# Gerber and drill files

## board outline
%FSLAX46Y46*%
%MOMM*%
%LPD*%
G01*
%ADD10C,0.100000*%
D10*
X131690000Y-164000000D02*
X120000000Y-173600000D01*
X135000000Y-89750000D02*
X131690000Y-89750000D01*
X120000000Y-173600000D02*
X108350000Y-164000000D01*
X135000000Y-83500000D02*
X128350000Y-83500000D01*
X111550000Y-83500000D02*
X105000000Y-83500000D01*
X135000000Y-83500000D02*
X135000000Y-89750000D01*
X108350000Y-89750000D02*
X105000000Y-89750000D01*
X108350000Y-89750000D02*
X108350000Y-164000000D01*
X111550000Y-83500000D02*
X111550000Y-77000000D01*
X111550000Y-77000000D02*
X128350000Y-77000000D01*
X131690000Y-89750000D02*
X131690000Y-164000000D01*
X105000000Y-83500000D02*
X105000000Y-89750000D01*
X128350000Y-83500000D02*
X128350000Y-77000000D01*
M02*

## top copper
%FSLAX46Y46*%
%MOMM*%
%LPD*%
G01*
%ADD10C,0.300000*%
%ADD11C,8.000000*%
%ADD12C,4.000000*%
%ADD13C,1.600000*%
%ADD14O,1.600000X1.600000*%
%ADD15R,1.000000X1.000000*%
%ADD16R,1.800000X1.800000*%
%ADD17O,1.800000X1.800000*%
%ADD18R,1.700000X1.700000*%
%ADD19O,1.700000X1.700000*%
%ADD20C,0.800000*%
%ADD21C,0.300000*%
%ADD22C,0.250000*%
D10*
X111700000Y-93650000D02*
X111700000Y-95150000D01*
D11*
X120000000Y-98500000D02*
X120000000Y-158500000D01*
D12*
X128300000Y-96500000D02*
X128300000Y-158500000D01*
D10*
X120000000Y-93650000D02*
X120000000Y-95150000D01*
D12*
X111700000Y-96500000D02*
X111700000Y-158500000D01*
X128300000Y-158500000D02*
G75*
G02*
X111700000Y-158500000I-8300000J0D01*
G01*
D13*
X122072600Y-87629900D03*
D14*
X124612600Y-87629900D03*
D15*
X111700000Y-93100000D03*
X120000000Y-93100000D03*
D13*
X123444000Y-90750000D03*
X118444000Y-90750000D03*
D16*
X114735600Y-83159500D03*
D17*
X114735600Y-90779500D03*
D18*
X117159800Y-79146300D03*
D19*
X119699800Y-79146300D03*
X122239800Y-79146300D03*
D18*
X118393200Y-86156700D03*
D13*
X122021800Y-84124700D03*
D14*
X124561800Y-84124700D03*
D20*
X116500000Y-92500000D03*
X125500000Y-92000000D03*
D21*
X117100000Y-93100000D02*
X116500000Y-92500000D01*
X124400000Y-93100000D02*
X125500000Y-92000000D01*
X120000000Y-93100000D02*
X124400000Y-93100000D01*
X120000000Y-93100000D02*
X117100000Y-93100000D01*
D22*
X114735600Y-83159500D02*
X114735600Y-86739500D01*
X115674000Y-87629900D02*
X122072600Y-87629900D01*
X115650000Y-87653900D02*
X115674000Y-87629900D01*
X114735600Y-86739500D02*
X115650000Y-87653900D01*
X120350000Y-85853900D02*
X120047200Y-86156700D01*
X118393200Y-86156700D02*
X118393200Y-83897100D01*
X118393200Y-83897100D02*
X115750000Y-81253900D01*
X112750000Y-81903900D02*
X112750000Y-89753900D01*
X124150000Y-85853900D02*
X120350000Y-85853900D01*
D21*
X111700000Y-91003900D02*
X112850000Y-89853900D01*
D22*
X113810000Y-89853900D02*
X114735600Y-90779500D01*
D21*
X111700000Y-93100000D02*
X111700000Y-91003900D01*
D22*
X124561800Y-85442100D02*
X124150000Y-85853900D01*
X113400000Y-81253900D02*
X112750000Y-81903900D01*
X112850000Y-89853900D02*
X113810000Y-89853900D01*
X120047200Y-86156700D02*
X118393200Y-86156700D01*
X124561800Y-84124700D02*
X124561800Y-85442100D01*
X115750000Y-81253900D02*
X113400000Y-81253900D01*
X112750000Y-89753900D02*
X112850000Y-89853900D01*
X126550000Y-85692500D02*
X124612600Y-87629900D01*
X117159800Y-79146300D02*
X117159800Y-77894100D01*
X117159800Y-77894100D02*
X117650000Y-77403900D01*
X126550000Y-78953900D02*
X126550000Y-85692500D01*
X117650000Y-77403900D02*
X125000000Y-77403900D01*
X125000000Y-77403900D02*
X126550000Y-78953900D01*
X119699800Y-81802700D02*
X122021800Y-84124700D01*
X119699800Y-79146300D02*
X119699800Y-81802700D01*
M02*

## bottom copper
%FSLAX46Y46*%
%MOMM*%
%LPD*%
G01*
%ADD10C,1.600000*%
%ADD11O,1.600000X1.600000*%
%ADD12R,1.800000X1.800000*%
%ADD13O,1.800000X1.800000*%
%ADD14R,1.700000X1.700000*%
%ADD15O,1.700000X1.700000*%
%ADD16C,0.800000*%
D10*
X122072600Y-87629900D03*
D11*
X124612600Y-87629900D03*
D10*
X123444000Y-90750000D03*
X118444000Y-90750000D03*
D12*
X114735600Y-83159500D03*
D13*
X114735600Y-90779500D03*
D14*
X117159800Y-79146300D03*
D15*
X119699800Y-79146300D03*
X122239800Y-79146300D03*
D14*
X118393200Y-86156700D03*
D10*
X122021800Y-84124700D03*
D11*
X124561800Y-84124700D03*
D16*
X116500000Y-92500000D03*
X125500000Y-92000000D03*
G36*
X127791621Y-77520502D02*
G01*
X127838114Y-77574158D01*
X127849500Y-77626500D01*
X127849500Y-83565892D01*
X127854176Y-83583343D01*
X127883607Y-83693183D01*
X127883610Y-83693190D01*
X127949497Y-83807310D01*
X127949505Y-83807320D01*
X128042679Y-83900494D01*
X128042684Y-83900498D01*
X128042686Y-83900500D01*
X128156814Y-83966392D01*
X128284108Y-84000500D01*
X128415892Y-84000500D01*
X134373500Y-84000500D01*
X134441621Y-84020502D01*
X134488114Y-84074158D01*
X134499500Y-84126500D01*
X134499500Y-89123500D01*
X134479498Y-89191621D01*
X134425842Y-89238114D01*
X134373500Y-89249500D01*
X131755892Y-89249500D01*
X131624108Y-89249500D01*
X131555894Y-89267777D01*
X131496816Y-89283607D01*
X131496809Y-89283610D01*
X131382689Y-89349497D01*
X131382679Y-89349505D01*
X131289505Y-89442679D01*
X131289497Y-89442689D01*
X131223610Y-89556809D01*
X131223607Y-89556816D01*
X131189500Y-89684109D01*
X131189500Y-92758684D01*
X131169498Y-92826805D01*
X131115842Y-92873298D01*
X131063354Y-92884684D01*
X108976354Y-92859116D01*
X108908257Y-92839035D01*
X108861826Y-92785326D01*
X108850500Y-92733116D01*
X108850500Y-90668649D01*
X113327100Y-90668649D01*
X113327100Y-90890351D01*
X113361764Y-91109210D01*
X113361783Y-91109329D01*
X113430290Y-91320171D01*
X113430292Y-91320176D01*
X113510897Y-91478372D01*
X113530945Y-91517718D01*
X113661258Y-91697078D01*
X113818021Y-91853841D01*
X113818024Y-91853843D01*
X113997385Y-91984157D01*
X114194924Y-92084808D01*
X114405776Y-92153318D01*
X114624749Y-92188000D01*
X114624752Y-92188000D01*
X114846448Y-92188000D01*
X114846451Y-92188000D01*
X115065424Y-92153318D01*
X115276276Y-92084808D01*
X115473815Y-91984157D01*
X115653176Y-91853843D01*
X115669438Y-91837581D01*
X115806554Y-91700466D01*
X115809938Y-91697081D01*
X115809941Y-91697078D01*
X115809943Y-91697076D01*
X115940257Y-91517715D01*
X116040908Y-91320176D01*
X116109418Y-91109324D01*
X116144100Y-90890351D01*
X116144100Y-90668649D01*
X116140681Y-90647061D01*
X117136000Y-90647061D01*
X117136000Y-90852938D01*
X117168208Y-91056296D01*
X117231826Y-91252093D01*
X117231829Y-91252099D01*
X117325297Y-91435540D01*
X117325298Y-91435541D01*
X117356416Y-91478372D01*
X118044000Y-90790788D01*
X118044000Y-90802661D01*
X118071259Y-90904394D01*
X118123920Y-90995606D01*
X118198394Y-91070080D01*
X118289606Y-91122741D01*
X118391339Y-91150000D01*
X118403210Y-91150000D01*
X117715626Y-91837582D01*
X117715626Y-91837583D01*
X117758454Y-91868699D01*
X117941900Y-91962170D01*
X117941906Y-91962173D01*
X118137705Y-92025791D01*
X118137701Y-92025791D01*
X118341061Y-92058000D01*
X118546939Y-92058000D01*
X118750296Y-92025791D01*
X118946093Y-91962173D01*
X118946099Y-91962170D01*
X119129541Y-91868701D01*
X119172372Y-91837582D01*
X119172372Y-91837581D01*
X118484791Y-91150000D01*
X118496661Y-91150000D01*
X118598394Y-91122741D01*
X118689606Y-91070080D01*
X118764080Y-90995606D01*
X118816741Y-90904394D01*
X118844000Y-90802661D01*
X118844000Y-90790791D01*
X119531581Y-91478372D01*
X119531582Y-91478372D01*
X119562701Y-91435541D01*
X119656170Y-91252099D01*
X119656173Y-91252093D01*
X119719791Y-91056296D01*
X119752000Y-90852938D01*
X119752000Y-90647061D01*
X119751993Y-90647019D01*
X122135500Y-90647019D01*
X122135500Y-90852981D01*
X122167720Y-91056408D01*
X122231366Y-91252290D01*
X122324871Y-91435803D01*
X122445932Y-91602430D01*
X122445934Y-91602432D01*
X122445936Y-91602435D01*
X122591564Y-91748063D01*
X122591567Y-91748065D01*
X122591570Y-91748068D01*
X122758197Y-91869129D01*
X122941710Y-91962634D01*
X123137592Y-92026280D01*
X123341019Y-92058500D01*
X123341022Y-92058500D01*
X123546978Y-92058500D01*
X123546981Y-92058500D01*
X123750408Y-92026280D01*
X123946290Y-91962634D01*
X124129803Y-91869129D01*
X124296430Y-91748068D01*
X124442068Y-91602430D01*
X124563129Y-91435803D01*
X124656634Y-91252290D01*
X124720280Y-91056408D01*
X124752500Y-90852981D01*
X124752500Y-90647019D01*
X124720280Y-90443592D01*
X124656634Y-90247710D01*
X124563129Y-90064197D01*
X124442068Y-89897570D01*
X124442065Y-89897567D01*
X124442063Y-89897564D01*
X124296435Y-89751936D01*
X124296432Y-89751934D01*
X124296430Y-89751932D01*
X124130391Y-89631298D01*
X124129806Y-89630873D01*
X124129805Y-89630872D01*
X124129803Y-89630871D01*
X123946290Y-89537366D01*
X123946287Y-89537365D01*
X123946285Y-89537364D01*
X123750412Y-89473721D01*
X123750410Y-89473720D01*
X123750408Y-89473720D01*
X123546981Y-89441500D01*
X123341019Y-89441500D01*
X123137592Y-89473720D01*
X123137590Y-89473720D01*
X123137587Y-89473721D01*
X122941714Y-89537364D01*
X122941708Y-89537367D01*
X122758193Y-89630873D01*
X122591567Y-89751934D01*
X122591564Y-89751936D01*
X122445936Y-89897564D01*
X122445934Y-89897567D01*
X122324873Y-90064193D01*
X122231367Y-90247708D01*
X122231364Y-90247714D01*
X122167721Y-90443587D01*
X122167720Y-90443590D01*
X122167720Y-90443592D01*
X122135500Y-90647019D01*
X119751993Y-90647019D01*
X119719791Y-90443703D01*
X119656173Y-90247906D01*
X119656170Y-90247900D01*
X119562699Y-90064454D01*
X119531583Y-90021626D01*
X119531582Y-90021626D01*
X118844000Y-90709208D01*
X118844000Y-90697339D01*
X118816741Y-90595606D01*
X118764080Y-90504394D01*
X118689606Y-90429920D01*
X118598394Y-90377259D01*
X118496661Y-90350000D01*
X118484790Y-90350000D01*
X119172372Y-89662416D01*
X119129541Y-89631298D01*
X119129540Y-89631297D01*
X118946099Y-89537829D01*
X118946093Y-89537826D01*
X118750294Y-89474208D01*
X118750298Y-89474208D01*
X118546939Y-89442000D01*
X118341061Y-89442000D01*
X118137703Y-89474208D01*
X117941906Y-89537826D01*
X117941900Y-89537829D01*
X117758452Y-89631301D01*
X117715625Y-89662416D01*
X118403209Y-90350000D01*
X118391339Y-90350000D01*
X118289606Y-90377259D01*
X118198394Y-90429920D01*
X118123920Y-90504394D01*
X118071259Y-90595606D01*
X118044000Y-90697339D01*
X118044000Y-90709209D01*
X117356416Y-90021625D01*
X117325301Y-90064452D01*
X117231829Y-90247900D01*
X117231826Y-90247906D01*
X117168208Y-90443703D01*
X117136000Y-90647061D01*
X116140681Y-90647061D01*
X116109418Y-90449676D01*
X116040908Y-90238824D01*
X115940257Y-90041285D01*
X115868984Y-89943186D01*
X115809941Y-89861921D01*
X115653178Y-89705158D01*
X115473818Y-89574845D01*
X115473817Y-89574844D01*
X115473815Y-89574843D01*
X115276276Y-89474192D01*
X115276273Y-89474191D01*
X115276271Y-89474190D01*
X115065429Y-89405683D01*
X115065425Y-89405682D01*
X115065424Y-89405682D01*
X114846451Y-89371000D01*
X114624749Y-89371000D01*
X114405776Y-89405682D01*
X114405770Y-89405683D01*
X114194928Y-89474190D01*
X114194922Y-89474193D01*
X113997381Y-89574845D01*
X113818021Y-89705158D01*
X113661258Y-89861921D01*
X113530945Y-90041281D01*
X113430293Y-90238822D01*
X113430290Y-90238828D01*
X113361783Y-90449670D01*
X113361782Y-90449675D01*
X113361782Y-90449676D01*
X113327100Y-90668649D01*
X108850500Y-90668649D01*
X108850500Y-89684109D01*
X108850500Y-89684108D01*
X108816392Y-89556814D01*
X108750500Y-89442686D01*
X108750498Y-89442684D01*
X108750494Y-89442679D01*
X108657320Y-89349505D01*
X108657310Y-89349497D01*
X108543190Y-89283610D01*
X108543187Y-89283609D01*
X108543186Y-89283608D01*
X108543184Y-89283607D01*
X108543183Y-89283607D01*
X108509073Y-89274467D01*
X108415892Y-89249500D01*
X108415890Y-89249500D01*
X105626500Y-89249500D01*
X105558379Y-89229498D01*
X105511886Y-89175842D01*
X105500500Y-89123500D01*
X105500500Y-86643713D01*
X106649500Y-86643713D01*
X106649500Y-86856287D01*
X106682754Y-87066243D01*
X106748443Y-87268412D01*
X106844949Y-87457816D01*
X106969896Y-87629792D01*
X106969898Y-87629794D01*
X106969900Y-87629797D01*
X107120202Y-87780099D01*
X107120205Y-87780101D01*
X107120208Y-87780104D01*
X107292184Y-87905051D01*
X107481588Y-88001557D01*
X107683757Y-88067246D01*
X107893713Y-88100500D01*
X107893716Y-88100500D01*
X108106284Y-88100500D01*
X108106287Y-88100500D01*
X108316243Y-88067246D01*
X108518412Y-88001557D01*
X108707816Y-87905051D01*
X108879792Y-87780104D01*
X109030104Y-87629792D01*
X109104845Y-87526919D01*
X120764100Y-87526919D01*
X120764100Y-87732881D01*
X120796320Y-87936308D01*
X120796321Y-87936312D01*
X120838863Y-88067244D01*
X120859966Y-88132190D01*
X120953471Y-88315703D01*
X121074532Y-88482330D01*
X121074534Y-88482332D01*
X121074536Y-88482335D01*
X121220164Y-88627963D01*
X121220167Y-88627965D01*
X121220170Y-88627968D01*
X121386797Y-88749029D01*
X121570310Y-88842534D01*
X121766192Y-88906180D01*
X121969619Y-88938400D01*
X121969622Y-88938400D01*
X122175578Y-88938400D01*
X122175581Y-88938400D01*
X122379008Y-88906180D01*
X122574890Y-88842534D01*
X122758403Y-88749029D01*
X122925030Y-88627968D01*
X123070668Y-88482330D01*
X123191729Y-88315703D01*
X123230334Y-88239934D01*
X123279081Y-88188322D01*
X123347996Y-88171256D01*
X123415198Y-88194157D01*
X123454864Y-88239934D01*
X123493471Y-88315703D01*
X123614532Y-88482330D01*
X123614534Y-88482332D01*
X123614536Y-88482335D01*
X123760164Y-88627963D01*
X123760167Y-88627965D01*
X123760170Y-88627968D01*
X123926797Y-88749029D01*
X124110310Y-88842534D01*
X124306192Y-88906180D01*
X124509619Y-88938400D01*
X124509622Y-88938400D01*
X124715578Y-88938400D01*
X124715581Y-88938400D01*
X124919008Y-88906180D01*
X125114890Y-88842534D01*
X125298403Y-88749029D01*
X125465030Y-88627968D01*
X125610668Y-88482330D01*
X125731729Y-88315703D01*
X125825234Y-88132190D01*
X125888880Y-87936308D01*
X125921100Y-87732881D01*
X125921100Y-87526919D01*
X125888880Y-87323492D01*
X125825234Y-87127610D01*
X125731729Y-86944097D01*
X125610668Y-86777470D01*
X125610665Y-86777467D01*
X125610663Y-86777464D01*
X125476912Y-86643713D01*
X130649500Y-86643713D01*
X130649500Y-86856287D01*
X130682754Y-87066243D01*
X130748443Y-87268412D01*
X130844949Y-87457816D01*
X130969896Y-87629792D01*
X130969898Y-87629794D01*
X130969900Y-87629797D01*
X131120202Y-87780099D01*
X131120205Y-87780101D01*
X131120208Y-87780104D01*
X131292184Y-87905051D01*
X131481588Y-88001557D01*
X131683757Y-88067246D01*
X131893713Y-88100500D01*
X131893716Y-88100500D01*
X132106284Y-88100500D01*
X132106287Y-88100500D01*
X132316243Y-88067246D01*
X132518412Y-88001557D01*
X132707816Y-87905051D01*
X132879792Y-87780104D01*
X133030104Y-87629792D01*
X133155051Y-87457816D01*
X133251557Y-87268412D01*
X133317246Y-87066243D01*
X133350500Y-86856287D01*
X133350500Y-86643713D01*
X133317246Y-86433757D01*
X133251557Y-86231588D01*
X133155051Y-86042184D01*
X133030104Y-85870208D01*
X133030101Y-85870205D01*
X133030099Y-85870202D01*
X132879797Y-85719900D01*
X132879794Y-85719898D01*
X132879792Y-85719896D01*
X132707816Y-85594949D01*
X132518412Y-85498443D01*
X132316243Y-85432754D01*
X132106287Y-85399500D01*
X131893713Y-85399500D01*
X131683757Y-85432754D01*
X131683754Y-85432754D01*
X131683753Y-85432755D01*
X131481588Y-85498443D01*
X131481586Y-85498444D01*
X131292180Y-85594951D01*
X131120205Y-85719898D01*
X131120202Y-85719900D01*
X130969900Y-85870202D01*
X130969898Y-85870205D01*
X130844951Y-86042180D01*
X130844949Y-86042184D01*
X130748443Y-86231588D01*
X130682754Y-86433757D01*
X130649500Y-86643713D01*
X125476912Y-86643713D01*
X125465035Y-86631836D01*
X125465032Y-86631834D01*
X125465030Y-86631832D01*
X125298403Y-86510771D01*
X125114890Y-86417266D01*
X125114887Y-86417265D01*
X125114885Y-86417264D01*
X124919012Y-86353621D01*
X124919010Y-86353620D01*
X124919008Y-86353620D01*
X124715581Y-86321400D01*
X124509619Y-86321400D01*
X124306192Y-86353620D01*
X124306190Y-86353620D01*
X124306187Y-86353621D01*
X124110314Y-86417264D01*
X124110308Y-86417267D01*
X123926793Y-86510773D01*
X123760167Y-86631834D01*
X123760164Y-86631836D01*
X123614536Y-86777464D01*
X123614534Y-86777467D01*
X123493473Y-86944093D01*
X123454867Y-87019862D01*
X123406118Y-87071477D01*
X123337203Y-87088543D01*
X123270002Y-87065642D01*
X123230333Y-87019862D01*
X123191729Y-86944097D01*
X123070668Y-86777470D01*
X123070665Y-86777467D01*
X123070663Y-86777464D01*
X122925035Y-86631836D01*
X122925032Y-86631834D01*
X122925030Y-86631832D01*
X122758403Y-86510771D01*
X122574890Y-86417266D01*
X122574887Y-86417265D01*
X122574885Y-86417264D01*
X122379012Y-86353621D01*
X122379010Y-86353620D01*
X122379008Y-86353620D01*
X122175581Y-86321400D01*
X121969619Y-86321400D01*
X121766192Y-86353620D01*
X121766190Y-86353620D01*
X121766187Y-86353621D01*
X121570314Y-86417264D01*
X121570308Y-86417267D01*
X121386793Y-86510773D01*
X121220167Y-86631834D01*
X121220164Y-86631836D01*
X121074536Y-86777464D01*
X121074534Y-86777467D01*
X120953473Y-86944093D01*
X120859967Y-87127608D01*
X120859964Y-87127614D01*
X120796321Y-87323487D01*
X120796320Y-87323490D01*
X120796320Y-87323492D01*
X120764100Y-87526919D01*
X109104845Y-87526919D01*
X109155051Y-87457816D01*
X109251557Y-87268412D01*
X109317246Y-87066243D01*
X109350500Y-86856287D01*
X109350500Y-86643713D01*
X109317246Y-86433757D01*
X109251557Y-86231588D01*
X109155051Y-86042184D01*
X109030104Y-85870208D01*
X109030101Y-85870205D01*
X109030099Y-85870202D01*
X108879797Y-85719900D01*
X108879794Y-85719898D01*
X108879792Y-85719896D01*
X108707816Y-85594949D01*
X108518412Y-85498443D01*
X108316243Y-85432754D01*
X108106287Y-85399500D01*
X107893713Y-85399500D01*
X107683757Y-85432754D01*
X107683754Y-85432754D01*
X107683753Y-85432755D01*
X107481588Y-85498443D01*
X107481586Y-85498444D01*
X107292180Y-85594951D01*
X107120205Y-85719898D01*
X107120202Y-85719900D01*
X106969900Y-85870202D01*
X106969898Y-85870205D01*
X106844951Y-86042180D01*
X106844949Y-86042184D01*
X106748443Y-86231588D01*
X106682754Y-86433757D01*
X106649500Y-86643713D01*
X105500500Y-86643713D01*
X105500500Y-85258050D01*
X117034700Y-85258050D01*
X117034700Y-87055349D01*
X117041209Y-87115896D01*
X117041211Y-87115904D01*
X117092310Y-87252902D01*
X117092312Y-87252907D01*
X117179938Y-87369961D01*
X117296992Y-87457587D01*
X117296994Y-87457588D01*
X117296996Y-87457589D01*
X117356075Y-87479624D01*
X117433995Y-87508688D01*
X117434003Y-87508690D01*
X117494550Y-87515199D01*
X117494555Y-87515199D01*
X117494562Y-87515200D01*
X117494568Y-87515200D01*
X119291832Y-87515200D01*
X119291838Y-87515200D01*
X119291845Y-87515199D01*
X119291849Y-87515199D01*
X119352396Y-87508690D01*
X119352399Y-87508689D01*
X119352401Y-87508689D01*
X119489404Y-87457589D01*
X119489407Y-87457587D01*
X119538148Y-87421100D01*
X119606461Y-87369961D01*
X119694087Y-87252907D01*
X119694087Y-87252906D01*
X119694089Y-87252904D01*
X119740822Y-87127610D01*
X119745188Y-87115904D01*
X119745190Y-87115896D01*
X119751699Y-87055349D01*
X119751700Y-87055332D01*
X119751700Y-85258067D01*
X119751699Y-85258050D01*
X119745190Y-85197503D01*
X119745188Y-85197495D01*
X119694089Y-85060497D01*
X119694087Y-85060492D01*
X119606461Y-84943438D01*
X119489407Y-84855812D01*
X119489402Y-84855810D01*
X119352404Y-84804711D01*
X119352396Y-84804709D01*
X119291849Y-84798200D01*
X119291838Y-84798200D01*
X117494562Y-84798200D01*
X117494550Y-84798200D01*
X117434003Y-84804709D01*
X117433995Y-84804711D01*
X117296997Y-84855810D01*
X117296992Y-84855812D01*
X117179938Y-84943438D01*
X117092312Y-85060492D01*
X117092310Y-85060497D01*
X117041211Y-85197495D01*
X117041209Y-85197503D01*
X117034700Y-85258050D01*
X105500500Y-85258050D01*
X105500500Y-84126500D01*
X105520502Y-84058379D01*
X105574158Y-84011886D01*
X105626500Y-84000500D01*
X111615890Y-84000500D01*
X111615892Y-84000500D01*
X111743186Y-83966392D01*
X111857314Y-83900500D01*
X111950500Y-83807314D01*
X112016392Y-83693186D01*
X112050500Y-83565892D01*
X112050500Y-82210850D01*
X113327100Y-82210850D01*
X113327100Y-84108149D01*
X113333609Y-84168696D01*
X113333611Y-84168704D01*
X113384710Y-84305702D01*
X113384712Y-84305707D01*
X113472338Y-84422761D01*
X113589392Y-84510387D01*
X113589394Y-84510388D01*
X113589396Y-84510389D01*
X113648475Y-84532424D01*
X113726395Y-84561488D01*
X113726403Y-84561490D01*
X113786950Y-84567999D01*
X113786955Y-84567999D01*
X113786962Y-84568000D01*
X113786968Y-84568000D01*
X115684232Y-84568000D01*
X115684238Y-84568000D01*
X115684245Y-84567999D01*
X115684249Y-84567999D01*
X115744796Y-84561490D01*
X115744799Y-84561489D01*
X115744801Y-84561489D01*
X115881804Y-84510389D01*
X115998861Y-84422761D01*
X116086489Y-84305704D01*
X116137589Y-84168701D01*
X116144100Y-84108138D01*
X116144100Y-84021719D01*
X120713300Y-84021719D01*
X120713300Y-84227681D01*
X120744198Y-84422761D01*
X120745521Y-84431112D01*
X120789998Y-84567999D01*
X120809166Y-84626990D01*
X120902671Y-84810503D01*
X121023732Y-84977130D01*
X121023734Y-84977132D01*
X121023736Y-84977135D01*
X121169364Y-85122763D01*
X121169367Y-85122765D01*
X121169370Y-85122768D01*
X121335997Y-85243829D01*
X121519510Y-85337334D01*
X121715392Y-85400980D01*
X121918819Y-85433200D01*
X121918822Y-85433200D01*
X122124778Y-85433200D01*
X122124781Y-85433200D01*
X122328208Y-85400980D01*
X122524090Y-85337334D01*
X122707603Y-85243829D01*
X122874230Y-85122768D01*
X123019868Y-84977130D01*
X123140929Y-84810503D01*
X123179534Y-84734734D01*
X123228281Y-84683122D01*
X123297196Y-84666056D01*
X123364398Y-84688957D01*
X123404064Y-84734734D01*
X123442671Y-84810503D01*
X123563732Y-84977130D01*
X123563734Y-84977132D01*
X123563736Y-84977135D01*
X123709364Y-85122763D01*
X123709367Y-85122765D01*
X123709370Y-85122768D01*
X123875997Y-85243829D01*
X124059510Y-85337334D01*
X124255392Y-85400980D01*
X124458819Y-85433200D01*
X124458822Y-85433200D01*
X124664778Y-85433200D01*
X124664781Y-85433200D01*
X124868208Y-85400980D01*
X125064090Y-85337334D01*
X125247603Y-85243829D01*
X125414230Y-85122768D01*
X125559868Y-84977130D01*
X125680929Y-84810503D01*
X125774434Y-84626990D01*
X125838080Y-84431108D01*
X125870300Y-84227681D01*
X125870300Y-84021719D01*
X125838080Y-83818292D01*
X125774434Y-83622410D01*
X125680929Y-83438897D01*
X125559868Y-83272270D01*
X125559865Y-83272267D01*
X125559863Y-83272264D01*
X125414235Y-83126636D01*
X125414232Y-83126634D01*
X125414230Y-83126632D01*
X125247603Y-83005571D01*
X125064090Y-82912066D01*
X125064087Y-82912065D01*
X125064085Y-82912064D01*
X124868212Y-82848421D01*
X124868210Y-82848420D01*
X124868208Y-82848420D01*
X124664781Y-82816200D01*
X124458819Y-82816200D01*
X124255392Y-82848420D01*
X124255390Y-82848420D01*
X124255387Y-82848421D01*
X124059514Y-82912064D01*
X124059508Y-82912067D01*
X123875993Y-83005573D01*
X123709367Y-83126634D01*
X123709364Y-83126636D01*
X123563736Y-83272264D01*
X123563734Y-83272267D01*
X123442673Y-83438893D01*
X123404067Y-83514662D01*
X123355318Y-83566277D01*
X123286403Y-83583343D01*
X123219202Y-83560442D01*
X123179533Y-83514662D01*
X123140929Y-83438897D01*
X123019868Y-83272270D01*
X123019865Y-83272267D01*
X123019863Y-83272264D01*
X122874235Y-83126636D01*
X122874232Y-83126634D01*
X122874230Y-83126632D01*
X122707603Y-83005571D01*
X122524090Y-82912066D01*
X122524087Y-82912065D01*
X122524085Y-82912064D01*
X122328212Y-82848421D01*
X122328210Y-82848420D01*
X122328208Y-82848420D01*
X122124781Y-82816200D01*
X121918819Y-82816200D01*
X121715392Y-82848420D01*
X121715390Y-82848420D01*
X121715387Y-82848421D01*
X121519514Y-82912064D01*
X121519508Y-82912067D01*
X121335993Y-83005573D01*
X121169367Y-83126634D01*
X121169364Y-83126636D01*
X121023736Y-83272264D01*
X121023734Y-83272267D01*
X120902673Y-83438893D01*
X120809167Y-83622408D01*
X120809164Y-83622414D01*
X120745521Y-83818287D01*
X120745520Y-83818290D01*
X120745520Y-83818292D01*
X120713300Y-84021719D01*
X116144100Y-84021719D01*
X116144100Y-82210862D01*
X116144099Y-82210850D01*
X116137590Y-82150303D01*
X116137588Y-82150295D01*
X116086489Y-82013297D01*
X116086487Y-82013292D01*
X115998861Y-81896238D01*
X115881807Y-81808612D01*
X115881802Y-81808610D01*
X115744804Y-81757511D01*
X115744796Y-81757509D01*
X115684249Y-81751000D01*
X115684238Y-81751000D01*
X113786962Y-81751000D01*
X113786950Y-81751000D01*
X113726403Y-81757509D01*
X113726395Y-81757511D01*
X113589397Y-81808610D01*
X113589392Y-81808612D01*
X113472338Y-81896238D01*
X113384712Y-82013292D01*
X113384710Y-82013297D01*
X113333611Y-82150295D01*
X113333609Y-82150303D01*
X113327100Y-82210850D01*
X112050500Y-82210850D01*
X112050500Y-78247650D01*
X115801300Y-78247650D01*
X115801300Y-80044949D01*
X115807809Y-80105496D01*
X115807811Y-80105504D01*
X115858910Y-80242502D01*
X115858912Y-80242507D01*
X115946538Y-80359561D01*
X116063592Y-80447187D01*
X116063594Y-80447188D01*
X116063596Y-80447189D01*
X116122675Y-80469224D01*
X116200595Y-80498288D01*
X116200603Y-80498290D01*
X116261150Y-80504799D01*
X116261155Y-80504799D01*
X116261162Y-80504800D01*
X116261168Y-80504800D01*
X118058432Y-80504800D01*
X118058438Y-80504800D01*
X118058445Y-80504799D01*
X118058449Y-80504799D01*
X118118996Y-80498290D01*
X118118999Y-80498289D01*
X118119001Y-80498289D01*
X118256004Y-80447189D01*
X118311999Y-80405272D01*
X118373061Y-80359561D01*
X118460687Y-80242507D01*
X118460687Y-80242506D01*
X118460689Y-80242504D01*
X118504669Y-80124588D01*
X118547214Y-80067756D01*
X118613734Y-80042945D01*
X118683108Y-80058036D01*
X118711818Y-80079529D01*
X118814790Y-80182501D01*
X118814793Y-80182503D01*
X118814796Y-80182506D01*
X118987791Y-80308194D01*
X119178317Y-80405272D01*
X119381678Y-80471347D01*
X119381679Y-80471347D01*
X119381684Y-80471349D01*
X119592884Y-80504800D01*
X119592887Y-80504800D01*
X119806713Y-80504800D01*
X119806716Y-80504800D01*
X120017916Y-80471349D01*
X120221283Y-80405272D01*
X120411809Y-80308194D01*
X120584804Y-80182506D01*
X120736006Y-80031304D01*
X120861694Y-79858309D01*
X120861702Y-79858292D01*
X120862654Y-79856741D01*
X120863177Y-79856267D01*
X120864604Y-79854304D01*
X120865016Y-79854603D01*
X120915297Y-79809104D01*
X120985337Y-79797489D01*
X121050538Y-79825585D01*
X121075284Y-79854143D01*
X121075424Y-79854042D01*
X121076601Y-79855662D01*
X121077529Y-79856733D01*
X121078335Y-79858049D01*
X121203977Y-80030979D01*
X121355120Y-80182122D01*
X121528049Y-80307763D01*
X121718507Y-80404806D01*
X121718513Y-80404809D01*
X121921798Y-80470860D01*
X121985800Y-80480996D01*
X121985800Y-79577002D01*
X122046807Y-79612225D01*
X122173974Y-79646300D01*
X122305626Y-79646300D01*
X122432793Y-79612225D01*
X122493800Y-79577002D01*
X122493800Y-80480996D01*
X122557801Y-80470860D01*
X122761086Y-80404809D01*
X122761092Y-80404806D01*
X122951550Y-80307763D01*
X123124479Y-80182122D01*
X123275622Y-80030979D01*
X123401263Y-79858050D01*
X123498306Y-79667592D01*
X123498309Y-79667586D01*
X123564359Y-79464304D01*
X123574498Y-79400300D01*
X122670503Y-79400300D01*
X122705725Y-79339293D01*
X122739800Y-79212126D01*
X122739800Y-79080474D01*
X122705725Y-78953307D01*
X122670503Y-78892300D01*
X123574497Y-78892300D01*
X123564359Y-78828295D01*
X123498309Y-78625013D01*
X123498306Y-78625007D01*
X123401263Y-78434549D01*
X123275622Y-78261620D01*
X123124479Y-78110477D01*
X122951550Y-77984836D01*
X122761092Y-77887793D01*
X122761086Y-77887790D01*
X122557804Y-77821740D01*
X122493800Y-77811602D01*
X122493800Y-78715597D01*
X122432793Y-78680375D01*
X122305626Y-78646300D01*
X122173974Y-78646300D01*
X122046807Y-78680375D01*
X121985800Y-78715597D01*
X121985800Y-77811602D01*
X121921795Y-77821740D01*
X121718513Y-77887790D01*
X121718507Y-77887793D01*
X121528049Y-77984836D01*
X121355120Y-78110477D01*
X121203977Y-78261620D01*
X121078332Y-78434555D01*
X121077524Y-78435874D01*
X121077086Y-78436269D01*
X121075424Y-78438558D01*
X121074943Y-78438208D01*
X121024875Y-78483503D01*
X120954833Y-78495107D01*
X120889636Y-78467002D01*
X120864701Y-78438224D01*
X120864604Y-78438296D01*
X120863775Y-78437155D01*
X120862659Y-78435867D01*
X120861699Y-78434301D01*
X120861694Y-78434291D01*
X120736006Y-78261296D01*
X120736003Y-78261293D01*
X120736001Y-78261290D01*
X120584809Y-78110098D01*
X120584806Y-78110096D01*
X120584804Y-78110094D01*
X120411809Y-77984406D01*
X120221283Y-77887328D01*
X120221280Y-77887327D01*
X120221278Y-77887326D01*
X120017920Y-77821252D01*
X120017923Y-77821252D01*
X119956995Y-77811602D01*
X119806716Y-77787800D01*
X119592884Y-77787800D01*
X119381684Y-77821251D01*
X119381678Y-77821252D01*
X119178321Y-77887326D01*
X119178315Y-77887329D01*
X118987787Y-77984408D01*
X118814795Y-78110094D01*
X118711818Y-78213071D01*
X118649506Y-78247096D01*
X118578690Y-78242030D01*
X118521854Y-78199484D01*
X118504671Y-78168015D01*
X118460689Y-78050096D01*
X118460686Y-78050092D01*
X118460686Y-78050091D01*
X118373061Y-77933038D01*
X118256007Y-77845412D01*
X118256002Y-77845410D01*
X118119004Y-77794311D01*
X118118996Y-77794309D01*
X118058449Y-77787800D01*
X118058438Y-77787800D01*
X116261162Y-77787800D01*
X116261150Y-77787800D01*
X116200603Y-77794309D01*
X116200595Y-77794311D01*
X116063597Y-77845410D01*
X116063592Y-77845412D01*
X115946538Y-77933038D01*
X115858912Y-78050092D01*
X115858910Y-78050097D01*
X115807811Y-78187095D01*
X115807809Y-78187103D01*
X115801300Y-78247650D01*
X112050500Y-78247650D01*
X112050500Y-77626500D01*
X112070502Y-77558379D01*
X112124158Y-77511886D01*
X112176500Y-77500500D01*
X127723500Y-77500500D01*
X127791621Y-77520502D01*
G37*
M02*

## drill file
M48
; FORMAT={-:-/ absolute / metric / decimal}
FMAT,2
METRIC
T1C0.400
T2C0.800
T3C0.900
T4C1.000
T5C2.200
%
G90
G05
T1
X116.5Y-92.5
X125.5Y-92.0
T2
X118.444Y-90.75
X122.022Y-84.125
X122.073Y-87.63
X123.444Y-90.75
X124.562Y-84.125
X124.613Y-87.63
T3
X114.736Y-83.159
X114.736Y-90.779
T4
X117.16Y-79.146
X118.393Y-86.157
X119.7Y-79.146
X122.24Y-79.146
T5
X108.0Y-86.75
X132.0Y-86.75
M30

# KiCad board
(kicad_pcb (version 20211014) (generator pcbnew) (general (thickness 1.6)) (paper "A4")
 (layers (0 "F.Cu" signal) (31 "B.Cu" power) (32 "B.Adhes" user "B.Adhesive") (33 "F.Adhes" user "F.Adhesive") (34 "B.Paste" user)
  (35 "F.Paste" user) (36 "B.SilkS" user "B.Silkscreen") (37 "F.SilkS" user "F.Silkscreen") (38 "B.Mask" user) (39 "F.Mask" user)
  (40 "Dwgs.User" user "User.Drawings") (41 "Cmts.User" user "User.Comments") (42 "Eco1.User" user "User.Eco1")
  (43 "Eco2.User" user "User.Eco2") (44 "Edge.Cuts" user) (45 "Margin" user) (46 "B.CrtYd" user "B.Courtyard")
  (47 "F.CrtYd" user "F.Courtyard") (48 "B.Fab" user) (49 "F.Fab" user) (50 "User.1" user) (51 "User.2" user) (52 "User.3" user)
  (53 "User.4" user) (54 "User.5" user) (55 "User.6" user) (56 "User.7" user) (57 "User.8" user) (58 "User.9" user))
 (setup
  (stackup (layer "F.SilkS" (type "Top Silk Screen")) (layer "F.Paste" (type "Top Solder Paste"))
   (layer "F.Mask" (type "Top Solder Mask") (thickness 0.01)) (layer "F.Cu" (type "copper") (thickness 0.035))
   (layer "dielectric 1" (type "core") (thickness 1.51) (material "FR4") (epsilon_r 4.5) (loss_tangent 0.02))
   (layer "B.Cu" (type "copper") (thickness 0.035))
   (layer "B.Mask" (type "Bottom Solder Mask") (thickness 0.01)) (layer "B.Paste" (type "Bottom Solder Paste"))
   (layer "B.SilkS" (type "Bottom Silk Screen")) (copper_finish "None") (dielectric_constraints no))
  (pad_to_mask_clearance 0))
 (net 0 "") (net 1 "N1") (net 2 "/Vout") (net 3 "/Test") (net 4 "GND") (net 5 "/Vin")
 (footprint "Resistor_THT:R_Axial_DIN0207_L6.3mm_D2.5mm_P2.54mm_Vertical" (layer "F.Cu") (at 122.0726 87.6299)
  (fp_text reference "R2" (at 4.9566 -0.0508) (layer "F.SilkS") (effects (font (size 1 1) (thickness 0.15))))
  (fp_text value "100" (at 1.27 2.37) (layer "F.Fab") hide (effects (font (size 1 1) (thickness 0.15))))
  (pad "1" thru_hole circle (at 0 0) (size 1.6 1.6) (drill 0.8) (layers *.Cu *.Mask) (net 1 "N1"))
  (pad "2" thru_hole oval (at 2.54 0) (size 1.6 1.6) (drill 0.8) (layers *.Cu *.Mask) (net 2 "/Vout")))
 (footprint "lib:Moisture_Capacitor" (layer "F.Cu") (at 120 95.5)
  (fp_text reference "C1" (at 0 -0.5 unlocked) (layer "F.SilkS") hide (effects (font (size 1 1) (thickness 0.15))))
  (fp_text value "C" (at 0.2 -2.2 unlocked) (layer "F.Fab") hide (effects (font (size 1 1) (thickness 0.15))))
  (fp_line (start -8.3 -1.85) (end -8.3 -0.35) (layer "F.Cu") (width 0.3)) (fp_line (start 0 3) (end 0 63) (layer "F.Cu") (width 8))
  (fp_line (start 8.3 1) (end 8.3 63) (layer "F.Cu") (width 4))
  (fp_line (start 0 -1.85) (end 0 -0.35) (layer "F.Cu") (width 0.3))
  (fp_line (start -8.3 1) (end -8.3 63) (layer "F.Cu") (width 4))
  (fp_arc (start 8.3 63) (mid 0 71.3) (end -8.3 63) (layer "F.Cu") (width 4))
  (pad "1" smd rect (at -8.3 -2.4) (size 1 1) (layers "F.Cu" "F.Paste" "F.Mask") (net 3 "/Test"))
  (pad "2" smd rect (at 0 -2.4) (size 1 1) (layers "F.Cu" "F.Paste" "F.Mask") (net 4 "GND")))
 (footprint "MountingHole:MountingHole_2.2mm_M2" (layer "F.Cu") (at 108 86.75)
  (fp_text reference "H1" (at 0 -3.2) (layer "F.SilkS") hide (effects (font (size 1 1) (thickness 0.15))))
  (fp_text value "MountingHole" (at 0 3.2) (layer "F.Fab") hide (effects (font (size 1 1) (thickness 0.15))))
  (pad "" np_thru_hole circle (at 0 0) (size 2.2 2.2) (drill 2.2) (layers *.Cu *.Mask)))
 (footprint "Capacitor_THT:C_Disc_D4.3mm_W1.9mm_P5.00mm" (layer "F.Cu") (at 123.444 90.75 180)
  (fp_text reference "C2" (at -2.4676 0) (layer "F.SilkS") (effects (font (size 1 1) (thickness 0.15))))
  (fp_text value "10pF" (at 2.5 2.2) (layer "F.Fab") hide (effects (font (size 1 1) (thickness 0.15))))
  (pad "1" thru_hole circle (at 0 0 180) (size 1.6 1.6) (drill 0.8) (layers *.Cu *.Mask) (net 2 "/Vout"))
  (pad "2" thru_hole circle (at 5 0 180) (size 1.6 1.6) (drill 0.8) (layers *.Cu *.Mask) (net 4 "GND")))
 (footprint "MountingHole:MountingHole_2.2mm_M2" (layer "F.Cu") (at 132 86.75)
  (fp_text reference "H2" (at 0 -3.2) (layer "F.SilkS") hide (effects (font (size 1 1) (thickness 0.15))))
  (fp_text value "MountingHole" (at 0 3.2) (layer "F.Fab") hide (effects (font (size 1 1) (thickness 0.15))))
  (pad "" np_thru_hole circle (at 0 0) (size 2.2 2.2) (drill 2.2) (layers *.Cu *.Mask)))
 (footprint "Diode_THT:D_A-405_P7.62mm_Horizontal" (layer "F.Cu") (at 114.7356 83.1595 -90)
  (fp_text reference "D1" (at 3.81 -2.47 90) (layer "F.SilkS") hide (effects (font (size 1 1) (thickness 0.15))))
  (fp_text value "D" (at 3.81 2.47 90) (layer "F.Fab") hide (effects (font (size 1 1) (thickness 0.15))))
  (pad "1" thru_hole rect (at 0 0 270) (size 1.8 1.8) (drill 0.9) (layers *.Cu *.Mask) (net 1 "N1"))
  (pad "2" thru_hole oval (at 7.62 0 270) (size 1.8 1.8) (drill 0.9) (layers *.Cu *.Mask) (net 3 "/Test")))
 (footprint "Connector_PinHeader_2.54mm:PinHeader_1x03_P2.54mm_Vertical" (layer "F.Cu") (at 117.1598 79.1463 90)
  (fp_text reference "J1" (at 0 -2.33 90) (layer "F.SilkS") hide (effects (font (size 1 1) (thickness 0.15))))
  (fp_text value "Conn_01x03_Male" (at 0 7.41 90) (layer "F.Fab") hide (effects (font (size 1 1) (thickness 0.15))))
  (pad "1" thru_hole rect (at 0 0 90) (size 1.7 1.7) (drill 1) (layers *.Cu *.Mask) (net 2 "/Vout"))
  (pad "2" thru_hole oval (at 0 2.54 90) (size 1.7 1.7) (drill 1) (layers *.Cu *.Mask) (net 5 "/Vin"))
  (pad "3" thru_hole oval (at 0 5.08 90) (size 1.7 1.7) (drill 1) (layers *.Cu *.Mask) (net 4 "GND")))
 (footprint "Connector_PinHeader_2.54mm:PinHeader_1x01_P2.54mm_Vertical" (layer "F.Cu") (at 118.3932 86.1567)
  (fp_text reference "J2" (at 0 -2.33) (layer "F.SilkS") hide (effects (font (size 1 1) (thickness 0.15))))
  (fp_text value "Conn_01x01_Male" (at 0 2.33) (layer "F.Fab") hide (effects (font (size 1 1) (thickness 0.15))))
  (pad "1" thru_hole rect (at 0 0) (size 1.7 1.7) (drill 1) (layers *.Cu *.Mask) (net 3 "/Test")))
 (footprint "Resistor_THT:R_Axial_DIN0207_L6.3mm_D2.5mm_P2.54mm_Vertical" (layer "F.Cu") (at 122.0218 84.1247)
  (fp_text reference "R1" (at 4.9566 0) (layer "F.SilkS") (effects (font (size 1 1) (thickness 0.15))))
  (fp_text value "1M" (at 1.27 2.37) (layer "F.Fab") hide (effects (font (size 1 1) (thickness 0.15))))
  (pad "1" thru_hole circle (at 0 0) (size 1.6 1.6) (drill 0.8) (layers *.Cu *.Mask) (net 5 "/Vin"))
  (pad "2" thru_hole oval (at 2.54 0) (size 1.6 1.6) (drill 0.8) (layers *.Cu *.Mask) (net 3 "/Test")))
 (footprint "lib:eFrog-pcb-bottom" (layer "B.Cu") (at 120 86.75 180)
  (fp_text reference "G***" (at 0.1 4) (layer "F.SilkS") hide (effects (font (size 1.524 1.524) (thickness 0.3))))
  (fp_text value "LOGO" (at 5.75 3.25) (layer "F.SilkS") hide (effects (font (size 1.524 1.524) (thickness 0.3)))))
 (gr_line (start 131.69 164) (end 120 173.6) (layer "Edge.Cuts") (width 0.1))
 (gr_line (start 135 89.75) (end 131.69 89.75) (layer "Edge.Cuts") (width 0.1))
 (gr_line (start 120 173.6) (end 108.35 164) (layer "Edge.Cuts") (width 0.1))
 (gr_line (start 135 83.5) (end 128.35 83.5) (layer "Edge.Cuts") (width 0.1))
 (gr_line (start 111.55 83.5) (end 105 83.5) (layer "Edge.Cuts") (width 0.1))
 (gr_line (start 135 83.5) (end 135 89.75) (layer "Edge.Cuts") (width 0.1))
 (gr_line (start 108.35 89.75) (end 105 89.75) (layer "Edge.Cuts") (width 0.1))
 (gr_line (start 108.35 89.75) (end 108.35 164) (layer "Edge.Cuts") (width 0.1))
 (gr_line (start 111.55 83.5) (end 111.55 77) (layer "Edge.Cuts") (width 0.1))
 (gr_line (start 111.55 77) (end 128.35 77) (layer "Edge.Cuts") (width 0.1))
 (gr_line (start 131.69 89.75) (end 131.69 164) (layer "Edge.Cuts") (width 0.1))
 (gr_line (start 105 83.5) (end 105 89.75) (layer "Edge.Cuts") (width 0.1))
 (gr_line (start 128.35 83.5) (end 128.35 77) (layer "Edge.Cuts") (width 0.1))
 (segment (start 117.1 93.1) (end 116.5 92.5) (width 0.3) (layer "F.Cu") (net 4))
 (segment (start 124.4 93.1) (end 125.5 92) (width 0.3) (layer "F.Cu") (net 4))
 (segment (start 120 93.1) (end 124.4 93.1) (width 0.3) (layer "F.Cu") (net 4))
 (segment (start 120 93.1) (end 117.1 93.1) (width 0.3) (layer "F.Cu") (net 4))
 (via (at 116.5 92.5) (size 0.8) (drill 0.4) (layers "F.Cu" "B.Cu") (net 4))
 (via (at 125.5 92) (size 0.8) (drill 0.4) (layers "F.Cu" "B.Cu") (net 4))
 (segment (start 114.7356 83.1595) (end 114.7356 86.7395) (width 0.25) (layer "F.Cu") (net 1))
 (segment (start 115.674 87.6299) (end 122.0726 87.6299) (width 0.25) (layer "F.Cu") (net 1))
 (segment (start 115.65 87.6539) (end 115.674 87.6299) (width 0.25) (layer "F.Cu") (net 1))
 (segment (start 114.7356 86.7395) (end 115.65 87.6539) (width 0.25) (layer "F.Cu") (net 1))
 (segment (start 120.35 85.8539) (end 120.0472 86.1567) (width 0.25) (layer "F.Cu") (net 3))
 (segment (start 118.3932 86.1567) (end 118.3932 83.8971) (width 0.25) (layer "F.Cu") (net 3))
 (segment (start 118.3932 83.8971) (end 115.75 81.2539) (width 0.25) (layer "F.Cu") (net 3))
 (segment (start 112.75 81.9039) (end 112.75 89.7539) (width 0.25) (layer "F.Cu") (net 3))
 (segment (start 124.15 85.8539) (end 120.35 85.8539) (width 0.25) (layer "F.Cu") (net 3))
 (segment (start 111.7 91.0039) (end 112.85 89.8539) (width 0.3) (layer "F.Cu") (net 3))
 (segment (start 113.81 89.8539) (end 114.7356 90.7795) (width 0.25) (layer "F.Cu") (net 3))
 (segment (start 111.7 93.1) (end 111.7 91.0039) (width 0.3) (layer "F.Cu") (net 3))
 (segment (start 124.5618 85.4421) (end 124.15 85.8539) (width 0.25) (layer "F.Cu") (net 3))
 (segment (start 113.4 81.2539) (end 112.75 81.9039) (width 0.25) (layer "F.Cu") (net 3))
 (segment (start 112.85 89.8539) (end 113.81 89.8539) (width 0.25) (layer "F.Cu") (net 3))
 (segment (start 120.0472 86.1567) (end 118.3932 86.1567) (width 0.25) (layer "F.Cu") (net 3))
 (segment (start 124.5618 84.1247) (end 124.5618 85.4421) (width 0.25) (layer "F.Cu") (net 3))
 (segment (start 115.75 81.2539) (end 113.4 81.2539) (width 0.25) (layer "F.Cu") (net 3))
 (segment (start 112.75 89.7539) (end 112.85 89.8539) (width 0.25) (layer "F.Cu") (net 3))
 (segment (start 126.55 85.6925) (end 124.6126 87.6299) (width 0.25) (layer "F.Cu") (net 2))
 (segment (start 117.1598 79.1463) (end 117.1598 77.8941) (width 0.25) (layer "F.Cu") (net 2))
 (segment (start 117.1598 77.8941) (end 117.65 77.4039) (width 0.25) (layer "F.Cu") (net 2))
 (segment (start 126.55 78.9539) (end 126.55 85.6925) (width 0.25) (layer "F.Cu") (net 2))
 (segment (start 117.65 77.4039) (end 125 77.4039) (width 0.25) (layer "F.Cu") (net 2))
 (segment (start 125 77.4039) (end 126.55 78.9539) (width 0.25) (layer "F.Cu") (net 2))
 (segment (start 119.6998 81.8027) (end 122.0218 84.1247) (width 0.25) (layer "F.Cu") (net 5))
 (segment (start 119.6998 79.1463) (end 119.6998 81.8027) (width 0.25) (layer "F.Cu") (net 5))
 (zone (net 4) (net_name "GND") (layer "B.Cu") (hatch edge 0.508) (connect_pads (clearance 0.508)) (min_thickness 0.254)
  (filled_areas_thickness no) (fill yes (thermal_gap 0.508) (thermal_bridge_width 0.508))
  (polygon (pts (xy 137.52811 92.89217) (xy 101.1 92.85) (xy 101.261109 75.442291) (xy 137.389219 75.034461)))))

